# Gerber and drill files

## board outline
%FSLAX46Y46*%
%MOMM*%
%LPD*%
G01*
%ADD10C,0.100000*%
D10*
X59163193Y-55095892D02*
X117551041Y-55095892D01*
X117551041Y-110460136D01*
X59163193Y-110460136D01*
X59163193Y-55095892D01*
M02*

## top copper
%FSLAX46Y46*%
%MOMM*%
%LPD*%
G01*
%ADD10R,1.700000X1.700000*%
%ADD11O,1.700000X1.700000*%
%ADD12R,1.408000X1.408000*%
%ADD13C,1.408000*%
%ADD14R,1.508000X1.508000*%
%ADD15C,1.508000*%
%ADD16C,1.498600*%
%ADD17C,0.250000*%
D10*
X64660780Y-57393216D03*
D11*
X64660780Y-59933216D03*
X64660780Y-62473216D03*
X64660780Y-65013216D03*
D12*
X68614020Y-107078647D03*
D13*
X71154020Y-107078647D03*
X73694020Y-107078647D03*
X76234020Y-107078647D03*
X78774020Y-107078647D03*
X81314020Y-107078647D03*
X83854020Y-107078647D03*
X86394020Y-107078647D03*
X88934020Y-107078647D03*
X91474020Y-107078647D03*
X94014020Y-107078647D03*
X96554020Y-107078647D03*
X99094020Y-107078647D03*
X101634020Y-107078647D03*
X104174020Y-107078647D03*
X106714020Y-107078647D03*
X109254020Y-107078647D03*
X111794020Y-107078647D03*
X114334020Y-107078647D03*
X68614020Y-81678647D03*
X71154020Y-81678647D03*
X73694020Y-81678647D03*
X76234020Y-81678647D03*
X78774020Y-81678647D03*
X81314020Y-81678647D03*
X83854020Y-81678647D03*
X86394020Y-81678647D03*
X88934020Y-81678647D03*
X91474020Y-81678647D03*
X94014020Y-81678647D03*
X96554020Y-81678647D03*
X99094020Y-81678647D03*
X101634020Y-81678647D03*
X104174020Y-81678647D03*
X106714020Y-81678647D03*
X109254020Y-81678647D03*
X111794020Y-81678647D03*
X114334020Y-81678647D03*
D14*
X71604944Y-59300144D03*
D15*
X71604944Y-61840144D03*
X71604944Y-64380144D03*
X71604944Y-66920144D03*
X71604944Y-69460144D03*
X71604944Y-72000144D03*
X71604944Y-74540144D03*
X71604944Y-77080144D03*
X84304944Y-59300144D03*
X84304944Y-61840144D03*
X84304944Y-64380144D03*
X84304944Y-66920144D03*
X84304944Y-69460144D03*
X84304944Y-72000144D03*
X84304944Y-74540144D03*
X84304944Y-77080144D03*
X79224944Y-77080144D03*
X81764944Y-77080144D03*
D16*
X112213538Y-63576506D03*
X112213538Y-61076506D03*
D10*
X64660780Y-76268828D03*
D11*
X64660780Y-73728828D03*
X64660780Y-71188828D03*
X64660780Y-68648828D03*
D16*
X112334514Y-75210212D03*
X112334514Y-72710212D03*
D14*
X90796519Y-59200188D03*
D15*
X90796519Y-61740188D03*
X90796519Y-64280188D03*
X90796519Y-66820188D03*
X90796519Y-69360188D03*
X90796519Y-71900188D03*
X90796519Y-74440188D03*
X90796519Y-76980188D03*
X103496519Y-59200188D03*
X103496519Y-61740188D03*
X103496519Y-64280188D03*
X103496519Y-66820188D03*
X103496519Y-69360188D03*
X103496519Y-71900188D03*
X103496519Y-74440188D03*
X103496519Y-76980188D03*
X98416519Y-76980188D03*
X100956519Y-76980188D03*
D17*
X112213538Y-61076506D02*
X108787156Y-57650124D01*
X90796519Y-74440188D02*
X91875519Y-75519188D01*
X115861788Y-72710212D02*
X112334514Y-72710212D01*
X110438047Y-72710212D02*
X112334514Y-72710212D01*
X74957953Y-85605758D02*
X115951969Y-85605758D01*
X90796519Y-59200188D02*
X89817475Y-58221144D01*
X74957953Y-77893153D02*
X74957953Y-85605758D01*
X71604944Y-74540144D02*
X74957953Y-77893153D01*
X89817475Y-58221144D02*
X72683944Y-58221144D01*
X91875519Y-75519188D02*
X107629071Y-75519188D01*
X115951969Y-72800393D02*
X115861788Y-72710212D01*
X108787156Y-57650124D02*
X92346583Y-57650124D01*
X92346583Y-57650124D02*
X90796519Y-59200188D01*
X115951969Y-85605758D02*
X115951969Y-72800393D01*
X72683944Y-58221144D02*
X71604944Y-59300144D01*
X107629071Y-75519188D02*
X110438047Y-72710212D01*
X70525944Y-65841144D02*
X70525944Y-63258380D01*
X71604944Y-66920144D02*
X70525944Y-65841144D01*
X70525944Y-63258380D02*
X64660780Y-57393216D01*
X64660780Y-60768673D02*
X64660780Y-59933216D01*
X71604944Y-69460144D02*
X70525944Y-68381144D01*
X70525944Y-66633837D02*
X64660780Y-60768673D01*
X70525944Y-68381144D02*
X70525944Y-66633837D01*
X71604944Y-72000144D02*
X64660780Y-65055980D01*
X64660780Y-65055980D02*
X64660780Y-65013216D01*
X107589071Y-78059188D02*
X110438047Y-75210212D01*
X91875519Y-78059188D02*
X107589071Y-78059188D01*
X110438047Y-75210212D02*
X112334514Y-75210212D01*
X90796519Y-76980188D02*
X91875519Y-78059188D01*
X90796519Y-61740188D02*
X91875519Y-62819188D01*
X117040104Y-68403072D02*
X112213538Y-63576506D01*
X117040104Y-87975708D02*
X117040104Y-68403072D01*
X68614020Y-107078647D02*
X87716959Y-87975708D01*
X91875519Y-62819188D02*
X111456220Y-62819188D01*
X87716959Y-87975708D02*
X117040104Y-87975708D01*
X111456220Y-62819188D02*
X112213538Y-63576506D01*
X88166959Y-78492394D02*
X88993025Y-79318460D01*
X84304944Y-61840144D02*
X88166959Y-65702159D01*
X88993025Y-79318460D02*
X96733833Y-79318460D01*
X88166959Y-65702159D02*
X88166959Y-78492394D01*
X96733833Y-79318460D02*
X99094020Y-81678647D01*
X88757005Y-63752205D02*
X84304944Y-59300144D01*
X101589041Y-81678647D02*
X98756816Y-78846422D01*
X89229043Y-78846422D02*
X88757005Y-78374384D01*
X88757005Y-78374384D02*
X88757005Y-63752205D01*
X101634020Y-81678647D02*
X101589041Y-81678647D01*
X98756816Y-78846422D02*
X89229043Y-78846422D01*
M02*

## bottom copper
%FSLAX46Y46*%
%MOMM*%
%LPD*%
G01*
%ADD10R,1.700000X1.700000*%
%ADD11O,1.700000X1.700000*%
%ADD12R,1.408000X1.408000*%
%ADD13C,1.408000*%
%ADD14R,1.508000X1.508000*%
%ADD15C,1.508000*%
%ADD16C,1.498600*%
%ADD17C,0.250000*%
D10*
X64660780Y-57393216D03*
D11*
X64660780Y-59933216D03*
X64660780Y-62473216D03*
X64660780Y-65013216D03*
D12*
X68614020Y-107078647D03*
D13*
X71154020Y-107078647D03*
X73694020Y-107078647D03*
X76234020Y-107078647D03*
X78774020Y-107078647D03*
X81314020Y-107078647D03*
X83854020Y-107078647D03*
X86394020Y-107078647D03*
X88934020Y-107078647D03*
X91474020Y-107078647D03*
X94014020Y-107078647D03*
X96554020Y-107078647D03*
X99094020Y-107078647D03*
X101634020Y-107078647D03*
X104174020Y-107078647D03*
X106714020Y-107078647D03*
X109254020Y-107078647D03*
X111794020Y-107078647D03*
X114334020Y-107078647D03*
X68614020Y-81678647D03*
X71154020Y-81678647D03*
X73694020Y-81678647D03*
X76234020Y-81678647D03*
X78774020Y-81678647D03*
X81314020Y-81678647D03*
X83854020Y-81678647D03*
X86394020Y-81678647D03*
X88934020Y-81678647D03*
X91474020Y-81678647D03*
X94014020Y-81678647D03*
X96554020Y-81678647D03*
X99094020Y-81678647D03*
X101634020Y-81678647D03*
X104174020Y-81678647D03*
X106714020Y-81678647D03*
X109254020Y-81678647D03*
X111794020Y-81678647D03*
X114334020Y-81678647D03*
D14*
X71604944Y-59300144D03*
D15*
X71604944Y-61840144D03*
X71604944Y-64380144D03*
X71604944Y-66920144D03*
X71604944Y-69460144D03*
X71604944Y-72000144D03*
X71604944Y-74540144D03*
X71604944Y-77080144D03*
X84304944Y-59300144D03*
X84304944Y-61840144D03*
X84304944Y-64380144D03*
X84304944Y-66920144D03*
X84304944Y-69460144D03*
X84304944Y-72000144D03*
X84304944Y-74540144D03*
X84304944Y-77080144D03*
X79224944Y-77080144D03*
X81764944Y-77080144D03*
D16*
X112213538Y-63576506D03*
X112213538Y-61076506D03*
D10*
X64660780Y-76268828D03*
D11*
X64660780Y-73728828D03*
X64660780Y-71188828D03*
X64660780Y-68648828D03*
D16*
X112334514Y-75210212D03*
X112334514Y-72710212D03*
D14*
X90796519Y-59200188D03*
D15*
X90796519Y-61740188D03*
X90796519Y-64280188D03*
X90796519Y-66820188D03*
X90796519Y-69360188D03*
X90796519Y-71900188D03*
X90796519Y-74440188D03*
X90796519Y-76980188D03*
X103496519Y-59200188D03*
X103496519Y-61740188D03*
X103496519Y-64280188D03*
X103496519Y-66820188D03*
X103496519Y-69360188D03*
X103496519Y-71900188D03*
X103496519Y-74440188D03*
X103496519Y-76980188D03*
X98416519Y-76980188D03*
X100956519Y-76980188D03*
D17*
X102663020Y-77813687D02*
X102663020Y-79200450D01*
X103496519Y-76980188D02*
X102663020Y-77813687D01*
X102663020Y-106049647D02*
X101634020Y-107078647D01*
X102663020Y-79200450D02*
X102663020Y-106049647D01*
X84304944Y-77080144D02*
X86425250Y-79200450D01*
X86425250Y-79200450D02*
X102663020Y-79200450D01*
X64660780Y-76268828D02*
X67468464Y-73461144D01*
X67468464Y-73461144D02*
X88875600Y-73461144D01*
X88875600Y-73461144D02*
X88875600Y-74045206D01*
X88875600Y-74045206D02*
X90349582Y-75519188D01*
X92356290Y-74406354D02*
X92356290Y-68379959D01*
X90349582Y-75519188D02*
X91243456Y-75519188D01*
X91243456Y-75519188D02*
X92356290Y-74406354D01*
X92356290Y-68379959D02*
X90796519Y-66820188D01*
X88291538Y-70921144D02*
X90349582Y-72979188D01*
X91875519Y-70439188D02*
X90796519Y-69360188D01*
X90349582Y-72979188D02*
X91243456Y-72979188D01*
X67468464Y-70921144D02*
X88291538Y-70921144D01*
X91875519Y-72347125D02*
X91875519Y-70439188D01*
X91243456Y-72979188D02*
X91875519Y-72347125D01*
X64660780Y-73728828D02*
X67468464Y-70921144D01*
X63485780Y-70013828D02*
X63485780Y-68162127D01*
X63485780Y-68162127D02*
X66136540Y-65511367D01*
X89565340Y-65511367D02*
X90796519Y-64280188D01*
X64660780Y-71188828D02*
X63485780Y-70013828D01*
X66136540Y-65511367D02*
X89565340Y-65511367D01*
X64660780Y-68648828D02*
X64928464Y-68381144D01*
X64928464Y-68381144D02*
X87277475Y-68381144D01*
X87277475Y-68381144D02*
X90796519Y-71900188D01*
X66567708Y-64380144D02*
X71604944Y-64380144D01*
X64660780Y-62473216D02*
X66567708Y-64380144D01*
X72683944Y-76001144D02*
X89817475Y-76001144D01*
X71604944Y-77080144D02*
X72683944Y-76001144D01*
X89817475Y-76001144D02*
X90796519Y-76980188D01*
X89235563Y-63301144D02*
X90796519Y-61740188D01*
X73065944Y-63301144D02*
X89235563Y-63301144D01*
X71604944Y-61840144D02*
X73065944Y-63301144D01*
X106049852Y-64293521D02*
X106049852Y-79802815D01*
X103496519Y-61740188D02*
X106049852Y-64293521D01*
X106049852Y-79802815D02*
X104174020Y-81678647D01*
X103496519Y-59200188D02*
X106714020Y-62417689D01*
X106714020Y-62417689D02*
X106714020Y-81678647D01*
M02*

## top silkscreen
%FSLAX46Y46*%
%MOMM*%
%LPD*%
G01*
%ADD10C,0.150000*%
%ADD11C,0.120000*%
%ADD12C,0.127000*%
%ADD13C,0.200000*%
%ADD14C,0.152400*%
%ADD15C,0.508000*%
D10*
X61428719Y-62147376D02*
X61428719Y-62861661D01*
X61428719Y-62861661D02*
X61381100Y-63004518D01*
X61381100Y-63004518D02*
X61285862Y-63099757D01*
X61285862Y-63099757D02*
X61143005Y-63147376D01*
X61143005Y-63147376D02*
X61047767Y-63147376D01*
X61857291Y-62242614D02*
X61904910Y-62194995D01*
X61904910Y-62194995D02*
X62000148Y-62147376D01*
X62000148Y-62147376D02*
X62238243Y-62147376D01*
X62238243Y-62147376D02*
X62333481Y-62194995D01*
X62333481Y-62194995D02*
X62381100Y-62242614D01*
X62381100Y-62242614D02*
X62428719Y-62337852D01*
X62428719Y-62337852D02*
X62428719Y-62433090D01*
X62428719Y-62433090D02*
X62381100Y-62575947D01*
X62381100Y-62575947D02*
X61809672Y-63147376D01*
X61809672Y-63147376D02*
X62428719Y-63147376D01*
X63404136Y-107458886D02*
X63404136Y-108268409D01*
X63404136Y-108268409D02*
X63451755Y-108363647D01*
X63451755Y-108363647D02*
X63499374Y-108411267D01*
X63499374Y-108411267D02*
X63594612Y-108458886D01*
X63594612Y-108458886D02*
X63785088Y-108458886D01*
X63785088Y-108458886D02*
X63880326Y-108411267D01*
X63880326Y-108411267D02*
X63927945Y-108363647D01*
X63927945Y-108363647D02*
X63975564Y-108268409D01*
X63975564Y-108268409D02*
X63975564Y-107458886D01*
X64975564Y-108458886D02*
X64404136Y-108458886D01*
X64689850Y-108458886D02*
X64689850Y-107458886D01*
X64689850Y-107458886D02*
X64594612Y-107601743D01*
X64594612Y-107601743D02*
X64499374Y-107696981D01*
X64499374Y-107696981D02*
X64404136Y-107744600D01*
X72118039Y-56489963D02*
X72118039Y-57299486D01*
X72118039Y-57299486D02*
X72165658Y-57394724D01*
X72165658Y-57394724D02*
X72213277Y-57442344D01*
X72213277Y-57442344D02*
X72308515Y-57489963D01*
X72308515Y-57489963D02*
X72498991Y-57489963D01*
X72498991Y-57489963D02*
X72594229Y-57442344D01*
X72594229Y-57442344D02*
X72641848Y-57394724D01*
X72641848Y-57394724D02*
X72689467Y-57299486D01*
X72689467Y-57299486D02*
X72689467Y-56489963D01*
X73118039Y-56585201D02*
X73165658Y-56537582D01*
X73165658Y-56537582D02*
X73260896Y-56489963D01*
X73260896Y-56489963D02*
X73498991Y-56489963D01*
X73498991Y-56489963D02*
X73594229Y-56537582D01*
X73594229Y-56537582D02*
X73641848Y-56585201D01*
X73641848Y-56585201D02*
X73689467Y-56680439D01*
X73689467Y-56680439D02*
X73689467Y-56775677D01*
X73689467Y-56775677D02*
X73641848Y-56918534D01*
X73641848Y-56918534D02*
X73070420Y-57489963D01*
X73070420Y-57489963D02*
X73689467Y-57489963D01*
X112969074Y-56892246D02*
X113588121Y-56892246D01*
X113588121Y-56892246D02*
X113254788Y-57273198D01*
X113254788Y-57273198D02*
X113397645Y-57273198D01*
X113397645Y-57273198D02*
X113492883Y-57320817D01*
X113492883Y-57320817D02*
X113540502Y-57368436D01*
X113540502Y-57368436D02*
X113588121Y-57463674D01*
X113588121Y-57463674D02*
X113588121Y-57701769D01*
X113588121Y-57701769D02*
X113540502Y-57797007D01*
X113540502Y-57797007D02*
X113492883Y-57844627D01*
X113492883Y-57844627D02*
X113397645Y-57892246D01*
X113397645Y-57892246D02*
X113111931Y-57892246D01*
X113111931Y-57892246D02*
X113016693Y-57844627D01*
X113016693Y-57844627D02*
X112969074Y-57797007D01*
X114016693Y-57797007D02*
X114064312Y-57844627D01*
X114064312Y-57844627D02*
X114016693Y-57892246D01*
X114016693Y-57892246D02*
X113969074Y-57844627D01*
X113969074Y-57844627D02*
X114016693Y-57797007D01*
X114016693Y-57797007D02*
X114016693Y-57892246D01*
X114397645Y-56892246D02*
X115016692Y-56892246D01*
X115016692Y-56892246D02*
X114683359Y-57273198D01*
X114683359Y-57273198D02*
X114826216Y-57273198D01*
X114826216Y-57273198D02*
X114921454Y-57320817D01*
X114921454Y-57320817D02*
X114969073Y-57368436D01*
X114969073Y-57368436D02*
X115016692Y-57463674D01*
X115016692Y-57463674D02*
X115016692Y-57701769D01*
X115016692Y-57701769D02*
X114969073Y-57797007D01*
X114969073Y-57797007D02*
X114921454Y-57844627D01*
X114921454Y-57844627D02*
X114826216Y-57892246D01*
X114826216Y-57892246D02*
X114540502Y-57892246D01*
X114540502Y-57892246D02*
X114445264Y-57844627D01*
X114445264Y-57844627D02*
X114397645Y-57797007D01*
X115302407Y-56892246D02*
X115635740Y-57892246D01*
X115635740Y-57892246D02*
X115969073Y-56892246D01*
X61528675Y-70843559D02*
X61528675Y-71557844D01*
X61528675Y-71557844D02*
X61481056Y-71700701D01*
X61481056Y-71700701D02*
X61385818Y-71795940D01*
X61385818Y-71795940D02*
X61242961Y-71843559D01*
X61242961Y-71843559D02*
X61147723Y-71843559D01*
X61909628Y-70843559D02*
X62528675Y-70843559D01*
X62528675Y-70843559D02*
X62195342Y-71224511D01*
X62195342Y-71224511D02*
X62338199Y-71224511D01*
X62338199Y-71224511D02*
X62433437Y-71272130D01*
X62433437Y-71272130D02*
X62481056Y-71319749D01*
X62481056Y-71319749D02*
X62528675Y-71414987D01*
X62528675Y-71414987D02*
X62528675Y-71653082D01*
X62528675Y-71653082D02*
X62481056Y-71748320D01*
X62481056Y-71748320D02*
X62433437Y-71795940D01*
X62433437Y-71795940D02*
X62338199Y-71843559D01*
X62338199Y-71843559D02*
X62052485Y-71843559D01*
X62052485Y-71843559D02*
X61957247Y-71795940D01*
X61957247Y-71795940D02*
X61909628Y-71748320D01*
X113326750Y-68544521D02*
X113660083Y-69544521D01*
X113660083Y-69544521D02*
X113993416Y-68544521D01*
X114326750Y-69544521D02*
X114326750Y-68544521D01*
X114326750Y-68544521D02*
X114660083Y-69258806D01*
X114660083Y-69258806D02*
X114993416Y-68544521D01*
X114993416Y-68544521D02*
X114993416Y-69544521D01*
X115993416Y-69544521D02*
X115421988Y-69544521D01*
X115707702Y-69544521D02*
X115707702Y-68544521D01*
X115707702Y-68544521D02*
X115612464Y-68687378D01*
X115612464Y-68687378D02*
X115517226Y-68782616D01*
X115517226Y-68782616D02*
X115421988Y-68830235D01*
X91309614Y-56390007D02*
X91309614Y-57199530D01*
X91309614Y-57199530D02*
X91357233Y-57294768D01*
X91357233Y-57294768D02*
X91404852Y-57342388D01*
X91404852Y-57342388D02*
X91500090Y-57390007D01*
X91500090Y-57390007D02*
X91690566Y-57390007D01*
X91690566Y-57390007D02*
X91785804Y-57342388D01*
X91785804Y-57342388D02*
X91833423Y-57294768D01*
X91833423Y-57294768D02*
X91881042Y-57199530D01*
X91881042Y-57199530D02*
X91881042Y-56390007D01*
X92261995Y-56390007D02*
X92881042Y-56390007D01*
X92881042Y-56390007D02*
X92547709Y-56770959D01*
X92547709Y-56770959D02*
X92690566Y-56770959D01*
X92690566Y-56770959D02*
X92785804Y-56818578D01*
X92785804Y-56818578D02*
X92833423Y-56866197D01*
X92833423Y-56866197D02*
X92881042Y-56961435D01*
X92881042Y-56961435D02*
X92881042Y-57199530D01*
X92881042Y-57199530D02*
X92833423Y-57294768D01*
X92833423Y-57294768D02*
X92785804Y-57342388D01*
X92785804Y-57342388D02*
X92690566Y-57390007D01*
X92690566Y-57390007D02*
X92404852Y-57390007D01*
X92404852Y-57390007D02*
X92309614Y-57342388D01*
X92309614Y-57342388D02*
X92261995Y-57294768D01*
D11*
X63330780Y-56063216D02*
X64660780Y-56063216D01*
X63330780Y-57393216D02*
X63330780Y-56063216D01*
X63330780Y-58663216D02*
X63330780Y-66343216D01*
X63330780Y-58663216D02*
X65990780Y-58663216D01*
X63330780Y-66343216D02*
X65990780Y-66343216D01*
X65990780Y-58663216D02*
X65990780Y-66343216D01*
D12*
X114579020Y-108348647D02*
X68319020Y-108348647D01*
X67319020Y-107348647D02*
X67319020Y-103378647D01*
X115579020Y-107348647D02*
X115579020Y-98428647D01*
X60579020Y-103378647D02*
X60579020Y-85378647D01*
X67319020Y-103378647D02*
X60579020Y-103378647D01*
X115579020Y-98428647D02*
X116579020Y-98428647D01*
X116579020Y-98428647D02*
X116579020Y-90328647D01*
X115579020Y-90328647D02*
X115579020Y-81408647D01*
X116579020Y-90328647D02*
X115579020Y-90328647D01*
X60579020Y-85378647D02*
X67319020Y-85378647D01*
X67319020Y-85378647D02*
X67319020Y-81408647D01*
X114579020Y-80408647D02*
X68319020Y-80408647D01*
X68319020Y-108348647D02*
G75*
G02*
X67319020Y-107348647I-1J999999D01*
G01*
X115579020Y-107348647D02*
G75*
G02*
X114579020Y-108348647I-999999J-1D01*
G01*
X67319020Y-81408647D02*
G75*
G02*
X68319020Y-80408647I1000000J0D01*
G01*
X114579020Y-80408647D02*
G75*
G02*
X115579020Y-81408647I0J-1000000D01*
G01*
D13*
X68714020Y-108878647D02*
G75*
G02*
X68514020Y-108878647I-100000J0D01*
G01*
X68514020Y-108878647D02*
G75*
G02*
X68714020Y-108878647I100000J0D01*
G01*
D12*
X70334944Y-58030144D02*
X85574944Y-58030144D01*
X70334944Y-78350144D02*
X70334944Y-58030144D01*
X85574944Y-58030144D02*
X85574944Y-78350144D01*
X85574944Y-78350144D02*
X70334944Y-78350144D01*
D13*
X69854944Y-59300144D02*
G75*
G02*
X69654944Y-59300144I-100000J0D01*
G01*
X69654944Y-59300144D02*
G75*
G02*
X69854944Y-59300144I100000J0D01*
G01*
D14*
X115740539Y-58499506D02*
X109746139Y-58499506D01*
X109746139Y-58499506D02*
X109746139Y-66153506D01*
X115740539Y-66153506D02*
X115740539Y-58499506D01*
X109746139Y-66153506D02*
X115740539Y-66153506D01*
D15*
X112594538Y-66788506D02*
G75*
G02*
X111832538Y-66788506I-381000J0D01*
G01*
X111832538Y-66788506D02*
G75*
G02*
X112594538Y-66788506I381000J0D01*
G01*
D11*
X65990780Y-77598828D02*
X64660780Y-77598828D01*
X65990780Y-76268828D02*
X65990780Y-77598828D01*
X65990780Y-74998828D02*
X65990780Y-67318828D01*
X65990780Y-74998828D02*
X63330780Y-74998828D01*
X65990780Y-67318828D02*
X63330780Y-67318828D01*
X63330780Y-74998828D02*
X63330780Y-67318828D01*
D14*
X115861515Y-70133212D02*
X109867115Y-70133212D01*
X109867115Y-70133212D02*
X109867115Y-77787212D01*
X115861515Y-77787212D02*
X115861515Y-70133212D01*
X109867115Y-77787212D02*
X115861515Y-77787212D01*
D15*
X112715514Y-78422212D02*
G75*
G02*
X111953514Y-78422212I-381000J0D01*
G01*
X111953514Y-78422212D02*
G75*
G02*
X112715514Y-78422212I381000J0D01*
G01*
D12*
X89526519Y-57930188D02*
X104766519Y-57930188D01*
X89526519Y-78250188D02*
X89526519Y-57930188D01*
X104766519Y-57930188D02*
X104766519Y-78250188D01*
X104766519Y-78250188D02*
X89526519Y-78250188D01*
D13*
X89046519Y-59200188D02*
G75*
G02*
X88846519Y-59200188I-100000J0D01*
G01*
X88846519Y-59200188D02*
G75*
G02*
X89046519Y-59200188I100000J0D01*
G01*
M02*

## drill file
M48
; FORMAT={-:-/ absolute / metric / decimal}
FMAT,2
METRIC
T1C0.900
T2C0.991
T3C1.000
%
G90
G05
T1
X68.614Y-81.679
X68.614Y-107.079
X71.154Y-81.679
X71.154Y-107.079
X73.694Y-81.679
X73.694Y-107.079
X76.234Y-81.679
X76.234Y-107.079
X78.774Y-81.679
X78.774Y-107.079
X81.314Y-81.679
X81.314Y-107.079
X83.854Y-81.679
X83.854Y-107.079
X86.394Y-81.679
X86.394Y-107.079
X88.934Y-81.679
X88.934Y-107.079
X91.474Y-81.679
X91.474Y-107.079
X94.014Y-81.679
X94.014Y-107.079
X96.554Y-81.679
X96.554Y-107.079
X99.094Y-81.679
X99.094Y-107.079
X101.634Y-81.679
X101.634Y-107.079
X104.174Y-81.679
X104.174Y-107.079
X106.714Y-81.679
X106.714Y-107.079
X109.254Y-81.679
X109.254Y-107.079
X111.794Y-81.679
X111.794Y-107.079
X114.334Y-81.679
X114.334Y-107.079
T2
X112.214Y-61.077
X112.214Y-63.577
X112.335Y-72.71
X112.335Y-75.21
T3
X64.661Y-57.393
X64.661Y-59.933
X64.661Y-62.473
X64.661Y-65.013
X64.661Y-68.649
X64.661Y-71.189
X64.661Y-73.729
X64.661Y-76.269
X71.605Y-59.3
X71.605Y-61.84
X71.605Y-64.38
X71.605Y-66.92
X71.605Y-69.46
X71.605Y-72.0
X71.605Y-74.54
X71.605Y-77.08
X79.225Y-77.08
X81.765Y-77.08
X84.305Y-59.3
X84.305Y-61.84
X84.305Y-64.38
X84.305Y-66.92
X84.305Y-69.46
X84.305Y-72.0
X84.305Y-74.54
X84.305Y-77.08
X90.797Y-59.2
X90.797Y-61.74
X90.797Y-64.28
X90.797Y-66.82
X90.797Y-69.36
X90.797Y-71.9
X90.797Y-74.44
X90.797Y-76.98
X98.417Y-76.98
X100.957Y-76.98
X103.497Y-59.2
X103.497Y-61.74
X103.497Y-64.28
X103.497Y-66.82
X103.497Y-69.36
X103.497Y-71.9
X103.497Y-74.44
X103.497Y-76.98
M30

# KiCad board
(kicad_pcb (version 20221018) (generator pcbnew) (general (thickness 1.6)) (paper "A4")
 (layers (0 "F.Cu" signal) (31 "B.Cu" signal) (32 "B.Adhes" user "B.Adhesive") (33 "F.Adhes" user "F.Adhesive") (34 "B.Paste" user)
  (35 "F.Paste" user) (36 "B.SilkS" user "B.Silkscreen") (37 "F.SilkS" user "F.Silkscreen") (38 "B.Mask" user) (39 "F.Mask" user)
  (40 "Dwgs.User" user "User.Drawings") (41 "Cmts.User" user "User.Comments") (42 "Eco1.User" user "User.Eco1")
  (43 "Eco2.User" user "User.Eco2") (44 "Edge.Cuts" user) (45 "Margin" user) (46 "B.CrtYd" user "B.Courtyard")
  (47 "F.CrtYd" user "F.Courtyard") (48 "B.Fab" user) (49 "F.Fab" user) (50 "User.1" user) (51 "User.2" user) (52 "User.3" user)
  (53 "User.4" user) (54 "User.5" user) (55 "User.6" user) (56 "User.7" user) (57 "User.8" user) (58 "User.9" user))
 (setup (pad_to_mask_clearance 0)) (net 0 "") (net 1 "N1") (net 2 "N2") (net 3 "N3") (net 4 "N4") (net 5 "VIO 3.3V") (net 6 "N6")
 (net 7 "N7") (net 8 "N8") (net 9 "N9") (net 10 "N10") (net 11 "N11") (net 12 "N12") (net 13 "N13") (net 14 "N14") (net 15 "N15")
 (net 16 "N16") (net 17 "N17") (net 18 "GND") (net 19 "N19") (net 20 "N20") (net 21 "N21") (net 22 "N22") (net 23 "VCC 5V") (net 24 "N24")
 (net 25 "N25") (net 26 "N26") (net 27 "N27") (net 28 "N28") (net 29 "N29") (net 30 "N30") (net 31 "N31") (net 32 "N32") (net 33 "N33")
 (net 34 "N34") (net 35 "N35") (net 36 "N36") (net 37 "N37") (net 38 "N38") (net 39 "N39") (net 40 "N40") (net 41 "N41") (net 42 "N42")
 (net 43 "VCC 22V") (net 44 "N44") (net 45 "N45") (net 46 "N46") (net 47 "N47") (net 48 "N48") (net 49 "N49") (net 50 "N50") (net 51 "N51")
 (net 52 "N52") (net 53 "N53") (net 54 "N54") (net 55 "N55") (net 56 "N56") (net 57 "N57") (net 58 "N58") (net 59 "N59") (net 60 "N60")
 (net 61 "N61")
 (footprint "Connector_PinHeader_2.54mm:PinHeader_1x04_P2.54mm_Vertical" (layer "F.Cu") (at 64.66078 57.393216)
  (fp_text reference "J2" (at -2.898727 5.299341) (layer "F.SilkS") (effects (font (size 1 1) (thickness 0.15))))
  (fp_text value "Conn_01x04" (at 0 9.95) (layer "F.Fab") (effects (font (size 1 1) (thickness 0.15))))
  (fp_line (start -1.33 -1.33) (end 0 -1.33) (stroke (width 0.12) (type solid)) (layer "F.SilkS"))
  (fp_line (start -1.33 0) (end -1.33 -1.33) (stroke (width 0.12) (type solid)) (layer "F.SilkS"))
  (fp_line (start -1.33 1.27) (end -1.33 8.95) (stroke (width 0.12) (type solid)) (layer "F.SilkS"))
  (fp_line (start -1.33 1.27) (end 1.33 1.27) (stroke (width 0.12) (type solid)) (layer "F.SilkS"))
  (fp_line (start -1.33 8.95) (end 1.33 8.95) (stroke (width 0.12) (type solid)) (layer "F.SilkS"))
  (fp_line (start 1.33 1.27) (end 1.33 8.95) (stroke (width 0.12) (type solid)) (layer "F.SilkS"))
  (pad "1" thru_hole rect (at 0 0) (size 1.7 1.7) (drill 1) (layers "*.Cu" "*.Mask") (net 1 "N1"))
  (pad "2" thru_hole oval (at 0 2.54) (size 1.7 1.7) (drill 1) (layers "*.Cu" "*.Mask") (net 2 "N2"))
  (pad "3" thru_hole oval (at 0 5.08) (size 1.7 1.7) (drill 1) (layers "*.Cu" "*.Mask") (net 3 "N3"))
  (pad "4" thru_hole oval (at 0 7.62) (size 1.7 1.7) (drill 1) (layers "*.Cu" "*.Mask") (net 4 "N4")))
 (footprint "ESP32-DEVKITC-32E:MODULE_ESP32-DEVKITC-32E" (layer "F.Cu") (at 91.44902 94.378647 90)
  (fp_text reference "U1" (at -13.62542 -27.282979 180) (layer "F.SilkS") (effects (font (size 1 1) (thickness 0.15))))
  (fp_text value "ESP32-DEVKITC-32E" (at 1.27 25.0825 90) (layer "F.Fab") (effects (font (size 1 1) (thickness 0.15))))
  (fp_line (start -13.97 23.13) (end -13.97 -23.13) (stroke (width 0.127) (type solid)) (layer "F.SilkS"))
  (fp_line (start -12.97 -24.13) (end -9 -24.13) (stroke (width 0.127) (type solid)) (layer "F.SilkS"))
  (fp_line (start -12.97 24.13) (end -4.05 24.13) (stroke (width 0.127) (type solid)) (layer "F.SilkS"))
  (fp_line (start -9 -30.87) (end 9 -30.87) (stroke (width 0.127) (type solid)) (layer "F.SilkS"))
  (fp_line (start -9 -24.13) (end -9 -30.87) (stroke (width 0.127) (type solid)) (layer "F.SilkS"))
  (fp_line (start -4.05 24.13) (end -4.05 25.13) (stroke (width 0.127) (type solid)) (layer "F.SilkS"))
  (fp_line (start -4.05 25.13) (end 4.05 25.13) (stroke (width 0.127) (type solid)) (layer "F.SilkS"))
  (fp_line (start 4.05 24.13) (end 12.97 24.13) (stroke (width 0.127) (type solid)) (layer "F.SilkS"))
  (fp_line (start 4.05 25.13) (end 4.05 24.13) (stroke (width 0.127) (type solid)) (layer "F.SilkS"))
  (fp_line (start 9 -30.87) (end 9 -24.13) (stroke (width 0.127) (type solid)) (layer "F.SilkS"))
  (fp_line (start 9 -24.13) (end 12.97 -24.13) (stroke (width 0.127) (type solid)) (layer "F.SilkS"))
  (fp_line (start 13.97 23.13) (end 13.97 -23.13) (stroke (width 0.127) (type solid)) (layer "F.SilkS"))
  (fp_arc (start -13.97 -23.13) (mid -13.677107 -23.837107) (end -12.97 -24.13) (stroke (width 0.127) (type solid)) (layer "F.SilkS"))
  (fp_arc (start -12.97 24.13) (mid -13.677107 23.837107) (end -13.97 23.13) (stroke (width 0.127) (type solid)) (layer "F.SilkS"))
  (fp_arc (start 12.97 -24.13) (mid 13.677107 -23.837107) (end 13.97 -23.13) (stroke (width 0.127) (type solid)) (layer "F.SilkS"))
  (fp_arc (start 13.97 23.13) (mid 13.677107 23.837107) (end 12.97 24.13) (stroke (width 0.127) (type solid)) (layer "F.SilkS"))
  (fp_circle (center -14.5 -22.835) (end -14.4 -22.835) (stroke (width 0.2) (type solid)) (fill none) (layer "F.SilkS"))
  (pad "J2_1" thru_hole rect (at -12.7 -22.835 90) (size 1.408 1.408) (drill 0.9) (layers "*.Cu" "*.Mask") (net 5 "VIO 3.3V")
   (solder_mask_margin 0.102))
  (pad "J2_2" thru_hole circle (at -12.7 -20.295 90) (size 1.408 1.408) (drill 0.9) (layers "*.Cu" "*.Mask") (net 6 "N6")
   (solder_mask_margin 0.102))
  (pad "J2_3" thru_hole circle (at -12.7 -17.755 90) (size 1.408 1.408) (drill 0.9) (layers "*.Cu" "*.Mask") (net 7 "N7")
   (solder_mask_margin 0.102))
  (pad "J2_4" thru_hole circle (at -12.7 -15.215 90) (size 1.408 1.408) (drill 0.9) (layers "*.Cu" "*.Mask") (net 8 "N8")
   (solder_mask_margin 0.102))
  (pad "J2_5" thru_hole circle (at -12.7 -12.675 90) (size 1.408 1.408) (drill 0.9) (layers "*.Cu" "*.Mask") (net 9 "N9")
   (solder_mask_margin 0.102))
  (pad "J2_6" thru_hole circle (at -12.7 -10.135 90) (size 1.408 1.408) (drill 0.9) (layers "*.Cu" "*.Mask") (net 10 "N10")
   (solder_mask_margin 0.102))
  (pad "J2_7" thru_hole circle (at -12.7 -7.595 90) (size 1.408 1.408) (drill 0.9) (layers "*.Cu" "*.Mask") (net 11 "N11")
   (solder_mask_margin 0.102))
  (pad "J2_8" thru_hole circle (at -12.7 -5.055 90) (size 1.408 1.408) (drill 0.9) (layers "*.Cu" "*.Mask") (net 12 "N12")
   (solder_mask_margin 0.102))
  (pad "J2_9" thru_hole circle (at -12.7 -2.515 90) (size 1.408 1.408) (drill 0.9) (layers "*.Cu" "*.Mask") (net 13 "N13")
   (solder_mask_margin 0.102))
  (pad "J2_10" thru_hole circle (at -12.7 0.025 90) (size 1.408 1.408) (drill 0.9) (layers "*.Cu" "*.Mask") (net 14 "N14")
   (solder_mask_margin 0.102))
  (pad "J2_11" thru_hole circle (at -12.7 2.565 90) (size 1.408 1.408) (drill 0.9) (layers "*.Cu" "*.Mask") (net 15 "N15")
   (solder_mask_margin 0.102))
  (pad "J2_12" thru_hole circle (at -12.7 5.105 90) (size 1.408 1.408) (drill 0.9) (layers "*.Cu" "*.Mask") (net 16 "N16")
   (solder_mask_margin 0.102))
  (pad "J2_13" thru_hole circle (at -12.7 7.645 90) (size 1.408 1.408) (drill 0.9) (layers "*.Cu" "*.Mask") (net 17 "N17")
   (solder_mask_margin 0.102))
  (pad "J2_14" thru_hole circle (at -12.7 10.185 90) (size 1.408 1.408) (drill 0.9) (layers "*.Cu" "*.Mask") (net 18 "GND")
   (solder_mask_margin 0.102))
  (pad "J2_15" thru_hole circle (at -12.7 12.725 90) (size 1.408 1.408) (drill 0.9) (layers "*.Cu" "*.Mask") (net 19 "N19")
   (solder_mask_margin 0.102))
  (pad "J2_16" thru_hole circle (at -12.7 15.265 90) (size 1.408 1.408) (drill 0.9) (layers "*.Cu" "*.Mask") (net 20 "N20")
   (solder_mask_margin 0.102))
  (pad "J2_17" thru_hole circle (at -12.7 17.805 90) (size 1.408 1.408) (drill 0.9) (layers "*.Cu" "*.Mask") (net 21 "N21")
   (solder_mask_margin 0.102))
  (pad "J2_18" thru_hole circle (at -12.7 20.345 90) (size 1.408 1.408) (drill 0.9) (layers "*.Cu" "*.Mask") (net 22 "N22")
   (solder_mask_margin 0.102))
  (pad "J2_19" thru_hole circle (at -12.7 22.885 90) (size 1.408 1.408) (drill 0.9) (layers "*.Cu" "*.Mask") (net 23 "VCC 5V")
   (solder_mask_margin 0.102))
  (pad "J3_1" thru_hole circle (at 12.7 -22.835 90) (size 1.408 1.408) (drill 0.9) (layers "*.Cu" "*.Mask") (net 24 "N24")
   (solder_mask_margin 0.102))
  (pad "J3_2" thru_hole circle (at 12.7 -20.295 90) (size 1.408 1.408) (drill 0.9) (layers "*.Cu" "*.Mask") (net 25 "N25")
   (solder_mask_margin 0.102))
  (pad "J3_3" thru_hole circle (at 12.7 -17.755 90) (size 1.408 1.408) (drill 0.9) (layers "*.Cu" "*.Mask") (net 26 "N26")
   (solder_mask_margin 0.102))
  (pad "J3_4" thru_hole circle (at 12.7 -15.215 90) (size 1.408 1.408) (drill 0.9) (layers "*.Cu" "*.Mask") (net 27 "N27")
   (solder_mask_margin 0.102))
  (pad "J3_5" thru_hole circle (at 12.7 -12.675 90) (size 1.408 1.408) (drill 0.9) (layers "*.Cu" "*.Mask") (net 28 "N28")
   (solder_mask_margin 0.102))
  (pad "J3_6" thru_hole circle (at 12.7 -10.135 90) (size 1.408 1.408) (drill 0.9) (layers "*.Cu" "*.Mask") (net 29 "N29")
   (solder_mask_margin 0.102))
  (pad "J3_7" thru_hole circle (at 12.7 -7.595 90) (size 1.408 1.408) (drill 0.9) (layers "*.Cu" "*.Mask") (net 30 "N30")
   (solder_mask_margin 0.102))
  (pad "J3_8" thru_hole circle (at 12.7 -5.055 90) (size 1.408 1.408) (drill 0.9) (layers "*.Cu" "*.Mask") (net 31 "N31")
   (solder_mask_margin 0.102))
  (pad "J3_9" thru_hole circle (at 12.7 -2.515 90) (size 1.408 1.408) (drill 0.9) (layers "*.Cu" "*.Mask") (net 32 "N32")
   (solder_mask_margin 0.102))
  (pad "J3_10" thru_hole circle (at 12.7 0.025 90) (size 1.408 1.408) (drill 0.9) (layers "*.Cu" "*.Mask") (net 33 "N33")
   (solder_mask_margin 0.102))
  (pad "J3_11" thru_hole circle (at 12.7 2.565 90) (size 1.408 1.408) (drill 0.9) (layers "*.Cu" "*.Mask") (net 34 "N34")
   (solder_mask_margin 0.102))
  (pad "J3_12" thru_hole circle (at 12.7 5.105 90) (size 1.408 1.408) (drill 0.9) (layers "*.Cu" "*.Mask") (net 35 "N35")
   (solder_mask_margin 0.102))
  (pad "J3_13" thru_hole circle (at 12.7 7.645 90) (size 1.408 1.408) (drill 0.9) (layers "*.Cu" "*.Mask") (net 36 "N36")
   (solder_mask_margin 0.102))
  (pad "J3_14" thru_hole circle (at 12.7 10.185 90) (size 1.408 1.408) (drill 0.9) (layers "*.Cu" "*.Mask") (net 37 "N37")
   (solder_mask_margin 0.102))
  (pad "J3_15" thru_hole circle (at 12.7 12.725 90) (size 1.408 1.408) (drill 0.9) (layers "*.Cu" "*.Mask") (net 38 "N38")
   (solder_mask_margin 0.102))
  (pad "J3_16" thru_hole circle (at 12.7 15.265 90) (size 1.408 1.408) (drill 0.9) (layers "*.Cu" "*.Mask") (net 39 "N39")
   (solder_mask_margin 0.102))
  (pad "J3_17" thru_hole circle (at 12.7 17.805 90) (size 1.408 1.408) (drill 0.9) (layers "*.Cu" "*.Mask") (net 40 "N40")
   (solder_mask_margin 0.102))
  (pad "J3_18" thru_hole circle (at 12.7 20.345 90) (size 1.408 1.408) (drill 0.9) (layers "*.Cu" "*.Mask") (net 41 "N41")
   (solder_mask_margin 0.102))
  (pad "J3_19" thru_hole circle (at 12.7 22.885 90) (size 1.408 1.408) (drill 0.9) (layers "*.Cu" "*.Mask") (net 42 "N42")
   (solder_mask_margin 0.102)))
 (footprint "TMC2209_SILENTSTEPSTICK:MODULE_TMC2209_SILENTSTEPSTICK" (layer "F.Cu") (at 77.954944 68.190144)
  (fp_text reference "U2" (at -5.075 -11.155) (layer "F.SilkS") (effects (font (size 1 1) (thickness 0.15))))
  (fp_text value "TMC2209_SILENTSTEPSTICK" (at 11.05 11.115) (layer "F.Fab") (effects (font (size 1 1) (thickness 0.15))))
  (fp_line (start -7.62 -10.16) (end 7.62 -10.16) (stroke (width 0.127) (type solid)) (layer "F.SilkS"))
  (fp_line (start -7.62 10.16) (end -7.62 -10.16) (stroke (width 0.127) (type solid)) (layer "F.SilkS"))
  (fp_line (start 7.62 -10.16) (end 7.62 10.16) (stroke (width 0.127) (type solid)) (layer "F.SilkS"))
  (fp_line (start 7.62 10.16) (end -7.62 10.16) (stroke (width 0.127) (type solid)) (layer "F.SilkS"))
  (fp_circle (center -8.2 -8.89) (end -8.1 -8.89) (stroke (width 0.2) (type solid)) (fill none) (layer "F.SilkS"))
  (pad "1" thru_hole rect (at -6.35 -8.89) (size 1.508 1.508) (drill 1) (layers "*.Cu" "*.Mask") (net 18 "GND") (solder_mask_margin 0.102))
  (pad "2" thru_hole circle (at -6.35 -6.35) (size 1.508 1.508) (drill 1) (layers "*.Cu" "*.Mask") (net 5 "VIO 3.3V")
   (solder_mask_margin 0.102))
  (pad "3" thru_hole circle (at -6.35 -3.81) (size 1.508 1.508) (drill 1) (layers "*.Cu" "*.Mask") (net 3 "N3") (solder_mask_margin 0.102))
  (pad "4" thru_hole circle (at -6.35 -1.27) (size 1.508 1.508) (drill 1) (layers "*.Cu" "*.Mask") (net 1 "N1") (solder_mask_margin 0.102))
  (pad "5" thru_hole circle (at -6.35 1.27) (size 1.508 1.508) (drill 1) (layers "*.Cu" "*.Mask") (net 2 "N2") (solder_mask_margin 0.102))
  (pad "6" thru_hole circle (at -6.35 3.81) (size 1.508 1.508) (drill 1) (layers "*.Cu" "*.Mask") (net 4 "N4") (solder_mask_margin 0.102))
  (pad "7" thru_hole circle (at -6.35 6.35) (size 1.508 1.508) (drill 1) (layers "*.Cu" "*.Mask") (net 18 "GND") (solder_mask_margin 0.102))
  (pad "8" thru_hole circle (at -6.35 8.89) (size 1.508 1.508) (drill 1) (layers "*.Cu" "*.Mask") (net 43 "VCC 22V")
   (solder_mask_margin 0.102))
  (pad "9" thru_hole circle (at 6.35 -8.89) (size 1.508 1.508) (drill 1) (layers "*.Cu" "*.Mask") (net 37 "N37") (solder_mask_margin 0.102))
  (pad "10" thru_hole circle (at 6.35 -6.35) (size 1.508 1.508) (drill 1) (layers "*.Cu" "*.Mask") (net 36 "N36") (solder_mask_margin 0.102))
  (pad "11" thru_hole circle (at 6.35 -3.81) (size 1.508 1.508) (drill 1) (layers "*.Cu" "*.Mask") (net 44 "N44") (solder_mask_margin 0.102))
  (pad "12" thru_hole circle (at 6.35 -1.27) (size 1.508 1.508) (drill 1) (layers "*.Cu" "*.Mask") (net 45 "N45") (solder_mask_margin 0.102))
  (pad "13" thru_hole circle (at 6.35 1.27) (size 1.508 1.508) (drill 1) (layers "*.Cu" "*.Mask") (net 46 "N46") (solder_mask_margin 0.102))
  (pad "14" thru_hole circle (at 6.35 3.81) (size 1.508 1.508) (drill 1) (layers "*.Cu" "*.Mask") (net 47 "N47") (solder_mask_margin 0.102))
  (pad "15" thru_hole circle (at 6.35 6.35) (size 1.508 1.508) (drill 1) (layers "*.Cu" "*.Mask") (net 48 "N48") (solder_mask_margin 0.102))
  (pad "16" thru_hole circle (at 6.35 8.89) (size 1.508 1.508) (drill 1) (layers "*.Cu" "*.Mask") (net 18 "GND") (solder_mask_margin 0.102))
  (pad "17" thru_hole circle (at 1.27 8.89) (size 1.508 1.508) (drill 1) (layers "*.Cu" "*.Mask") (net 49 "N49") (solder_mask_margin 0.102))
  (pad "18" thru_hole circle (at 3.81 8.89) (size 1.508 1.508) (drill 1) (layers "*.Cu" "*.Mask") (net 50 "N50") (solder_mask_margin 0.102)))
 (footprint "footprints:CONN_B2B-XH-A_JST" (layer "F.Cu") (at 112.213538 63.576506 -90)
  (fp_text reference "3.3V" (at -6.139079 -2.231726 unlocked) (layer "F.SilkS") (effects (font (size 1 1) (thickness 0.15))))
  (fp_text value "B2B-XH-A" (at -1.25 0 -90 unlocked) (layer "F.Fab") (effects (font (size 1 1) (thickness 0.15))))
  (fp_line (start -5.077 -3.527001) (end -5.077 2.467399) (stroke (width 0.1524) (type solid)) (layer "F.SilkS"))
  (fp_line (start -5.077 2.467399) (end 2.577 2.467399) (stroke (width 0.1524) (type solid)) (layer "F.SilkS"))
  (fp_line (start 2.577 -3.527001) (end -5.077 -3.527001) (stroke (width 0.1524) (type solid)) (layer "F.SilkS"))
  (fp_line (start 2.577 2.467399) (end 2.577 -3.527001) (stroke (width 0.1524) (type solid)) (layer "F.SilkS"))
  (fp_circle (center 3.212 0) (end 3.593 0) (stroke (width 0.508) (type solid)) (fill none) (layer "F.SilkS"))
  (pad "1" thru_hole circle (at 0 0 270) (size 1.4986 1.4986) (drill 0.9906) (layers "*.Cu" "*.Mask") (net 5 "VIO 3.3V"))
  (pad "2" thru_hole circle (at -2.5 0 270) (size 1.4986 1.4986) (drill 0.9906) (layers "*.Cu" "*.Mask") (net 18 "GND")))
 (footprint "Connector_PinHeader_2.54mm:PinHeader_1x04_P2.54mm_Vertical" (layer "F.Cu") (at 64.66078 76.268828 180)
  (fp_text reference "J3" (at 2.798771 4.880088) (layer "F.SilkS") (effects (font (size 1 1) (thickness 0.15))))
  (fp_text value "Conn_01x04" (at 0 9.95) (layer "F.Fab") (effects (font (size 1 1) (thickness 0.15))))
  (fp_line (start -1.33 -1.33) (end 0 -1.33) (stroke (width 0.12) (type solid)) (layer "F.SilkS"))
  (fp_line (start -1.33 0) (end -1.33 -1.33) (stroke (width 0.12) (type solid)) (layer "F.SilkS"))
  (fp_line (start -1.33 1.27) (end -1.33 8.95) (stroke (width 0.12) (type solid)) (layer "F.SilkS"))
  (fp_line (start -1.33 1.27) (end 1.33 1.27) (stroke (width 0.12) (type solid)) (layer "F.SilkS"))
  (fp_line (start -1.33 8.95) (end 1.33 8.95) (stroke (width 0.12) (type solid)) (layer "F.SilkS"))
  (fp_line (start 1.33 1.27) (end 1.33 8.95) (stroke (width 0.12) (type solid)) (layer "F.SilkS"))
  (pad "1" thru_hole rect (at 0 0 180) (size 1.7 1.7) (drill 1) (layers "*.Cu" "*.Mask") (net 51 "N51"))
  (pad "2" thru_hole oval (at 0 2.54 180) (size 1.7 1.7) (drill 1) (layers "*.Cu" "*.Mask") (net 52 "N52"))
  (pad "3" thru_hole oval (at 0 5.08 180) (size 1.7 1.7) (drill 1) (layers "*.Cu" "*.Mask") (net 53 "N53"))
  (pad "4" thru_hole oval (at 0 7.62 180) (size 1.7 1.7) (drill 1) (layers "*.Cu" "*.Mask") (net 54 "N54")))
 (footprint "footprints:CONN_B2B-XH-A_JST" (layer "F.Cu") (at 112.334514 75.210212 -90)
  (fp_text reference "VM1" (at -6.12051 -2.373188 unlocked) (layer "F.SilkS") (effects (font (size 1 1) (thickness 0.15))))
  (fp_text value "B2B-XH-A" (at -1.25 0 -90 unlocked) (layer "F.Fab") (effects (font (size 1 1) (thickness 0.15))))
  (fp_line (start -5.077 -3.527001) (end -5.077 2.467399) (stroke (width 0.1524) (type solid)) (layer "F.SilkS"))
  (fp_line (start -5.077 2.467399) (end 2.577 2.467399) (stroke (width 0.1524) (type solid)) (layer "F.SilkS"))
  (fp_line (start 2.577 -3.527001) (end -5.077 -3.527001) (stroke (width 0.1524) (type solid)) (layer "F.SilkS"))
  (fp_line (start 2.577 2.467399) (end 2.577 -3.527001) (stroke (width 0.1524) (type solid)) (layer "F.SilkS"))
  (fp_circle (center 3.212 0) (end 3.593 0) (stroke (width 0.508) (type solid)) (fill none) (layer "F.SilkS"))
  (pad "1" thru_hole circle (at 0 0 270) (size 1.4986 1.4986) (drill 0.9906) (layers "*.Cu" "*.Mask") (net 43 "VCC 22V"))
  (pad "2" thru_hole circle (at -2.5 0 270) (size 1.4986 1.4986) (drill 0.9906) (layers "*.Cu" "*.Mask") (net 18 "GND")))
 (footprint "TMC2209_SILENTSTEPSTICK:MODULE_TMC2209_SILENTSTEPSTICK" (layer "F.Cu") (at 97.146519 68.090188)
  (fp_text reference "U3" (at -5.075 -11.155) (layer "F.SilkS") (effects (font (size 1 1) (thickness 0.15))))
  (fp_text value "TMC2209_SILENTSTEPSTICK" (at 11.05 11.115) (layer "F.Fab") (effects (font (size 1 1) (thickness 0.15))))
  (fp_line (start -7.62 -10.16) (end 7.62 -10.16) (stroke (width 0.127) (type solid)) (layer "F.SilkS"))
  (fp_line (start -7.62 10.16) (end -7.62 -10.16) (stroke (width 0.127) (type solid)) (layer "F.SilkS"))
  (fp_line (start 7.62 -10.16) (end 7.62 10.16) (stroke (width 0.127) (type solid)) (layer "F.SilkS"))
  (fp_line (start 7.62 10.16) (end -7.62 10.16) (stroke (width 0.127) (type solid)) (layer "F.SilkS"))
  (fp_circle (center -8.2 -8.89) (end -8.1 -8.89) (stroke (width 0.2) (type solid)) (fill none) (layer "F.SilkS"))
  (pad "1" thru_hole rect (at -6.35 -8.89) (size 1.508 1.508) (drill 1) (layers "*.Cu" "*.Mask") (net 18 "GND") (solder_mask_margin 0.102))
  (pad "2" thru_hole circle (at -6.35 -6.35) (size 1.508 1.508) (drill 1) (layers "*.Cu" "*.Mask") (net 5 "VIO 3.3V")
   (solder_mask_margin 0.102))
  (pad "3" thru_hole circle (at -6.35 -3.81) (size 1.508 1.508) (drill 1) (layers "*.Cu" "*.Mask") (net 53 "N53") (solder_mask_margin 0.102))
  (pad "4" thru_hole circle (at -6.35 -1.27) (size 1.508 1.508) (drill 1) (layers "*.Cu" "*.Mask") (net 51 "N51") (solder_mask_margin 0.102))
  (pad "5" thru_hole circle (at -6.35 1.27) (size 1.508 1.508) (drill 1) (layers "*.Cu" "*.Mask") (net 52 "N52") (solder_mask_margin 0.102))
  (pad "6" thru_hole circle (at -6.35 3.81) (size 1.508 1.508) (drill 1) (layers "*.Cu" "*.Mask") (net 54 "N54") (solder_mask_margin 0.102))
  (pad "7" thru_hole circle (at -6.35 6.35) (size 1.508 1.508) (drill 1) (layers "*.Cu" "*.Mask") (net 18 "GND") (solder_mask_margin 0.102))
  (pad "8" thru_hole circle (at -6.35 8.89) (size 1.508 1.508) (drill 1) (layers "*.Cu" "*.Mask") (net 43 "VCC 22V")
   (solder_mask_margin 0.102))
  (pad "9" thru_hole circle (at 6.35 -8.89) (size 1.508 1.508) (drill 1) (layers "*.Cu" "*.Mask") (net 39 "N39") (solder_mask_margin 0.102))
  (pad "10" thru_hole circle (at 6.35 -6.35) (size 1.508 1.508) (drill 1) (layers "*.Cu" "*.Mask") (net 38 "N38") (solder_mask_margin 0.102))
  (pad "11" thru_hole circle (at 6.35 -3.81) (size 1.508 1.508) (drill 1) (layers "*.Cu" "*.Mask") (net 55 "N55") (solder_mask_margin 0.102))
  (pad "12" thru_hole circle (at 6.35 -1.27) (size 1.508 1.508) (drill 1) (layers "*.Cu" "*.Mask") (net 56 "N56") (solder_mask_margin 0.102))
  (pad "13" thru_hole circle (at 6.35 1.27) (size 1.508 1.508) (drill 1) (layers "*.Cu" "*.Mask") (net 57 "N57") (solder_mask_margin 0.102))
  (pad "14" thru_hole circle (at 6.35 3.81) (size 1.508 1.508) (drill 1) (layers "*.Cu" "*.Mask") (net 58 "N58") (solder_mask_margin 0.102))
  (pad "15" thru_hole circle (at 6.35 6.35) (size 1.508 1.508) (drill 1) (layers "*.Cu" "*.Mask") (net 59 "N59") (solder_mask_margin 0.102))
  (pad "16" thru_hole circle (at 6.35 8.89) (size 1.508 1.508) (drill 1) (layers "*.Cu" "*.Mask") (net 18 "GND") (solder_mask_margin 0.102))
  (pad "17" thru_hole circle (at 1.27 8.89) (size 1.508 1.508) (drill 1) (layers "*.Cu" "*.Mask") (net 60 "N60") (solder_mask_margin 0.102))
  (pad "18" thru_hole circle (at 3.81 8.89) (size 1.508 1.508) (drill 1) (layers "*.Cu" "*.Mask") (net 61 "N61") (solder_mask_margin 0.102)))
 (gr_rect (start 59.163193 55.095892) (end 117.551041 110.460136) (stroke (width 0.1) (type default)) (fill none) (layer "Edge.Cuts"))
 (segment (start 112.213538 61.076506) (end 108.787156 57.650124) (width 0.25) (layer "F.Cu") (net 18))
 (segment (start 90.796519 74.440188) (end 91.875519 75.519188) (width 0.25) (layer "F.Cu") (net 18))
 (segment (start 115.861788 72.710212) (end 112.334514 72.710212) (width 0.25) (layer "F.Cu") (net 18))
 (segment (start 110.438047 72.710212) (end 112.334514 72.710212) (width 0.25) (layer "F.Cu") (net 18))
 (segment (start 74.957953 85.605758) (end 115.951969 85.605758) (width 0.25) (layer "F.Cu") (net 18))
 (segment (start 90.796519 59.200188) (end 89.817475 58.221144) (width 0.25) (layer "F.Cu") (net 18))
 (segment (start 74.957953 77.893153) (end 74.957953 85.605758) (width 0.25) (layer "F.Cu") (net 18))
 (segment (start 71.604944 74.540144) (end 74.957953 77.893153) (width 0.25) (layer "F.Cu") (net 18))
 (segment (start 89.817475 58.221144) (end 72.683944 58.221144) (width 0.25) (layer "F.Cu") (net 18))
 (segment (start 91.875519 75.519188) (end 107.629071 75.519188) (width 0.25) (layer "F.Cu") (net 18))
 (segment (start 115.951969 72.800393) (end 115.861788 72.710212) (width 0.25) (layer "F.Cu") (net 18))
 (segment (start 108.787156 57.650124) (end 92.346583 57.650124) (width 0.25) (layer "F.Cu") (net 18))
 (segment (start 92.346583 57.650124) (end 90.796519 59.200188) (width 0.25) (layer "F.Cu") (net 18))
 (segment (start 115.951969 85.605758) (end 115.951969 72.800393) (width 0.25) (layer "F.Cu") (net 18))
 (segment (start 72.683944 58.221144) (end 71.604944 59.300144) (width 0.25) (layer "F.Cu") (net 18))
 (segment (start 107.629071 75.519188) (end 110.438047 72.710212) (width 0.25) (layer "F.Cu") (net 18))
 (segment (start 102.66302 77.813687) (end 102.66302 79.20045) (width 0.25) (layer "B.Cu") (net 18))
 (segment (start 103.496519 76.980188) (end 102.66302 77.813687) (width 0.25) (layer "B.Cu") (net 18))
 (segment (start 102.66302 106.049647) (end 101.63402 107.078647) (width 0.25) (layer "B.Cu") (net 18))
 (segment (start 102.66302 79.20045) (end 102.66302 106.049647) (width 0.25) (layer "B.Cu") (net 18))
 (segment (start 84.304944 77.080144) (end 86.42525 79.20045) (width 0.25) (layer "B.Cu") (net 18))
 (segment (start 86.42525 79.20045) (end 102.66302 79.20045) (width 0.25) (layer "B.Cu") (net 18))
 (segment (start 64.66078 76.268828) (end 67.468464 73.461144) (width 0.25) (layer "B.Cu") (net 51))
 (segment (start 67.468464 73.461144) (end 88.8756 73.461144) (width 0.25) (layer "B.Cu") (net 51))
 (segment (start 88.8756 73.461144) (end 88.8756 74.045206) (width 0.25) (layer "B.Cu") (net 51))
 (segment (start 88.8756 74.045206) (end 90.349582 75.519188) (width 0.25) (layer "B.Cu") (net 51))
 (segment (start 92.35629 74.406354) (end 92.35629 68.379959) (width 0.25) (layer "B.Cu") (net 51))
 (segment (start 90.349582 75.519188) (end 91.243456 75.519188) (width 0.25) (layer "B.Cu") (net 51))
 (segment (start 91.243456 75.519188) (end 92.35629 74.406354) (width 0.25) (layer "B.Cu") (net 51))
 (segment (start 92.35629 68.379959) (end 90.796519 66.820188) (width 0.25) (layer "B.Cu") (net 51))
 (segment (start 88.291538 70.921144) (end 90.349582 72.979188) (width 0.25) (layer "B.Cu") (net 52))
 (segment (start 91.875519 70.439188) (end 90.796519 69.360188) (width 0.25) (layer "B.Cu") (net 52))
 (segment (start 90.349582 72.979188) (end 91.243456 72.979188) (width 0.25) (layer "B.Cu") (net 52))
 (segment (start 67.468464 70.921144) (end 88.291538 70.921144) (width 0.25) (layer "B.Cu") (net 52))
 (segment (start 91.875519 72.347125) (end 91.875519 70.439188) (width 0.25) (layer "B.Cu") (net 52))
 (segment (start 91.243456 72.979188) (end 91.875519 72.347125) (width 0.25) (layer "B.Cu") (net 52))
 (segment (start 64.66078 73.728828) (end 67.468464 70.921144) (width 0.25) (layer "B.Cu") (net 52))
 (segment (start 63.48578 70.013828) (end 63.48578 68.162127) (width 0.25) (layer "B.Cu") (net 53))
 (segment (start 63.48578 68.162127) (end 66.13654 65.511367) (width 0.25) (layer "B.Cu") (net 53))
 (segment (start 89.56534 65.511367) (end 90.796519 64.280188) (width 0.25) (layer "B.Cu") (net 53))
 (segment (start 64.66078 71.188828) (end 63.48578 70.013828) (width 0.25) (layer "B.Cu") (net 53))
 (segment (start 66.13654 65.511367) (end 89.56534 65.511367) (width 0.25) (layer "B.Cu") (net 53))
 (segment (start 64.66078 68.648828) (end 64.928464 68.381144) (width 0.25) (layer "B.Cu") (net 54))
 (segment (start 64.928464 68.381144) (end 87.277475 68.381144) (width 0.25) (layer "B.Cu") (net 54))
 (segment (start 87.277475 68.381144) (end 90.796519 71.900188) (width 0.25) (layer "B.Cu") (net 54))
 (segment (start 70.525944 65.841144) (end 70.525944 63.25838) (width 0.25) (layer "F.Cu") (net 1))
 (segment (start 71.604944 66.920144) (end 70.525944 65.841144) (width 0.25) (layer "F.Cu") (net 1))
 (segment (start 70.525944 63.25838) (end 64.66078 57.393216) (width 0.25) (layer "F.Cu") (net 1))
 (segment (start 64.66078 60.768673) (end 64.66078 59.933216) (width 0.25) (layer "F.Cu") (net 2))
 (segment (start 71.604944 69.460144) (end 70.525944 68.381144) (width 0.25) (layer "F.Cu") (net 2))
 (segment (start 70.525944 66.633837) (end 64.66078 60.768673) (width 0.25) (layer "F.Cu") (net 2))
 (segment (start 70.525944 68.381144) (end 70.525944 66.633837) (width 0.25) (layer "F.Cu") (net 2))
 (segment (start 66.567708 64.380144) (end 71.604944 64.380144) (width 0.25) (layer "B.Cu") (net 3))
 (segment (start 64.66078 62.473216) (end 66.567708 64.380144) (width 0.25) (layer "B.Cu") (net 3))
 (segment (start 71.604944 72.000144) (end 64.66078 65.05598) (width 0.25) (layer "F.Cu") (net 4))
 (segment (start 64.66078 65.05598) (end 64.66078 65.013216) (width 0.25) (layer "F.Cu") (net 4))
 (segment (start 107.589071 78.059188) (end 110.438047 75.210212) (width 0.25) (layer "F.Cu") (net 43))
 (segment (start 91.875519 78.059188) (end 107.589071 78.059188) (width 0.25) (layer "F.Cu") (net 43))
 (segment (start 110.438047 75.210212) (end 112.334514 75.210212) (width 0.25) (layer "F.Cu") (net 43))
 (segment (start 90.796519 76.980188) (end 91.875519 78.059188) (width 0.25) (layer "F.Cu") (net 43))
 (segment (start 72.683944 76.001144) (end 89.817475 76.001144) (width 0.25) (layer "B.Cu") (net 43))
 (segment (start 71.604944 77.080144) (end 72.683944 76.001144) (width 0.25) (layer "B.Cu") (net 43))
 (segment (start 89.817475 76.001144) (end 90.796519 76.980188) (width 0.25) (layer "B.Cu") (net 43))
 (segment (start 90.796519 61.740188) (end 91.875519 62.819188) (width 0.25) (layer "F.Cu") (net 5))
 (segment (start 117.040104 68.403072) (end 112.213538 63.576506) (width 0.25) (layer "F.Cu") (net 5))
 (segment (start 117.040104 87.975708) (end 117.040104 68.403072) (width 0.25) (layer "F.Cu") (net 5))
 (segment (start 68.61402 107.078647) (end 87.716959 87.975708) (width 0.25) (layer "F.Cu") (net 5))
 (segment (start 91.875519 62.819188) (end 111.45622 62.819188) (width 0.25) (layer "F.Cu") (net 5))
 (segment (start 87.716959 87.975708) (end 117.040104 87.975708) (width 0.25) (layer "F.Cu") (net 5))
 (segment (start 111.45622 62.819188) (end 112.213538 63.576506) (width 0.25) (layer "F.Cu") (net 5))
 (segment (start 89.235563 63.301144) (end 90.796519 61.740188) (width 0.25) (layer "B.Cu") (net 5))
 (segment (start 73.065944 63.301144) (end 89.235563 63.301144) (width 0.25) (layer "B.Cu") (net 5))
 (segment (start 71.604944 61.840144) (end 73.065944 63.301144) (width 0.25) (layer "B.Cu") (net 5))
 (segment (start 88.166959 78.492394) (end 88.993025 79.31846) (width 0.25) (layer "F.Cu") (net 36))
 (segment (start 84.304944 61.840144) (end 88.166959 65.702159) (width 0.25) (layer "F.Cu") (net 36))
 (segment (start 88.993025 79.31846) (end 96.733833 79.31846) (width 0.25) (layer "F.Cu") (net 36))
 (segment (start 88.166959 65.702159) (end 88.166959 78.492394) (width 0.25) (layer "F.Cu") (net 36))
 (segment (start 96.733833 79.31846) (end 99.09402 81.678647) (width 0.25) (layer "F.Cu") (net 36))
 (segment (start 88.757005 63.752205) (end 84.304944 59.300144) (width 0.25) (layer "F.Cu") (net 37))
 (segment (start 101.589041 81.678647) (end 98.756816 78.846422) (width 0.25) (layer "F.Cu") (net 37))
 (segment (start 89.229043 78.846422) (end 88.757005 78.374384) (width 0.25) (layer "F.Cu") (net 37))
 (segment (start 88.757005 78.374384) (end 88.757005 63.752205) (width 0.25) (layer "F.Cu") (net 37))
 (segment (start 101.63402 81.678647) (end 101.589041 81.678647) (width 0.25) (layer "F.Cu") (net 37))
 (segment (start 98.756816 78.846422) (end 89.229043 78.846422) (width 0.25) (layer "F.Cu") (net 37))
 (segment (start 106.049852 64.293521) (end 106.049852 79.802815) (width 0.25) (layer "B.Cu") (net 38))
 (segment (start 103.496519 61.740188) (end 106.049852 64.293521) (width 0.25) (layer "B.Cu") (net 38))
 (segment (start 106.049852 79.802815) (end 104.17402 81.678647) (width 0.25) (layer "B.Cu") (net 38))
 (segment (start 103.496519 59.200188) (end 106.71402 62.417689) (width 0.25) (layer "B.Cu") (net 39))
 (segment (start 106.71402 62.417689) (end 106.71402 81.678647) (width 0.25) (layer "B.Cu") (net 39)))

